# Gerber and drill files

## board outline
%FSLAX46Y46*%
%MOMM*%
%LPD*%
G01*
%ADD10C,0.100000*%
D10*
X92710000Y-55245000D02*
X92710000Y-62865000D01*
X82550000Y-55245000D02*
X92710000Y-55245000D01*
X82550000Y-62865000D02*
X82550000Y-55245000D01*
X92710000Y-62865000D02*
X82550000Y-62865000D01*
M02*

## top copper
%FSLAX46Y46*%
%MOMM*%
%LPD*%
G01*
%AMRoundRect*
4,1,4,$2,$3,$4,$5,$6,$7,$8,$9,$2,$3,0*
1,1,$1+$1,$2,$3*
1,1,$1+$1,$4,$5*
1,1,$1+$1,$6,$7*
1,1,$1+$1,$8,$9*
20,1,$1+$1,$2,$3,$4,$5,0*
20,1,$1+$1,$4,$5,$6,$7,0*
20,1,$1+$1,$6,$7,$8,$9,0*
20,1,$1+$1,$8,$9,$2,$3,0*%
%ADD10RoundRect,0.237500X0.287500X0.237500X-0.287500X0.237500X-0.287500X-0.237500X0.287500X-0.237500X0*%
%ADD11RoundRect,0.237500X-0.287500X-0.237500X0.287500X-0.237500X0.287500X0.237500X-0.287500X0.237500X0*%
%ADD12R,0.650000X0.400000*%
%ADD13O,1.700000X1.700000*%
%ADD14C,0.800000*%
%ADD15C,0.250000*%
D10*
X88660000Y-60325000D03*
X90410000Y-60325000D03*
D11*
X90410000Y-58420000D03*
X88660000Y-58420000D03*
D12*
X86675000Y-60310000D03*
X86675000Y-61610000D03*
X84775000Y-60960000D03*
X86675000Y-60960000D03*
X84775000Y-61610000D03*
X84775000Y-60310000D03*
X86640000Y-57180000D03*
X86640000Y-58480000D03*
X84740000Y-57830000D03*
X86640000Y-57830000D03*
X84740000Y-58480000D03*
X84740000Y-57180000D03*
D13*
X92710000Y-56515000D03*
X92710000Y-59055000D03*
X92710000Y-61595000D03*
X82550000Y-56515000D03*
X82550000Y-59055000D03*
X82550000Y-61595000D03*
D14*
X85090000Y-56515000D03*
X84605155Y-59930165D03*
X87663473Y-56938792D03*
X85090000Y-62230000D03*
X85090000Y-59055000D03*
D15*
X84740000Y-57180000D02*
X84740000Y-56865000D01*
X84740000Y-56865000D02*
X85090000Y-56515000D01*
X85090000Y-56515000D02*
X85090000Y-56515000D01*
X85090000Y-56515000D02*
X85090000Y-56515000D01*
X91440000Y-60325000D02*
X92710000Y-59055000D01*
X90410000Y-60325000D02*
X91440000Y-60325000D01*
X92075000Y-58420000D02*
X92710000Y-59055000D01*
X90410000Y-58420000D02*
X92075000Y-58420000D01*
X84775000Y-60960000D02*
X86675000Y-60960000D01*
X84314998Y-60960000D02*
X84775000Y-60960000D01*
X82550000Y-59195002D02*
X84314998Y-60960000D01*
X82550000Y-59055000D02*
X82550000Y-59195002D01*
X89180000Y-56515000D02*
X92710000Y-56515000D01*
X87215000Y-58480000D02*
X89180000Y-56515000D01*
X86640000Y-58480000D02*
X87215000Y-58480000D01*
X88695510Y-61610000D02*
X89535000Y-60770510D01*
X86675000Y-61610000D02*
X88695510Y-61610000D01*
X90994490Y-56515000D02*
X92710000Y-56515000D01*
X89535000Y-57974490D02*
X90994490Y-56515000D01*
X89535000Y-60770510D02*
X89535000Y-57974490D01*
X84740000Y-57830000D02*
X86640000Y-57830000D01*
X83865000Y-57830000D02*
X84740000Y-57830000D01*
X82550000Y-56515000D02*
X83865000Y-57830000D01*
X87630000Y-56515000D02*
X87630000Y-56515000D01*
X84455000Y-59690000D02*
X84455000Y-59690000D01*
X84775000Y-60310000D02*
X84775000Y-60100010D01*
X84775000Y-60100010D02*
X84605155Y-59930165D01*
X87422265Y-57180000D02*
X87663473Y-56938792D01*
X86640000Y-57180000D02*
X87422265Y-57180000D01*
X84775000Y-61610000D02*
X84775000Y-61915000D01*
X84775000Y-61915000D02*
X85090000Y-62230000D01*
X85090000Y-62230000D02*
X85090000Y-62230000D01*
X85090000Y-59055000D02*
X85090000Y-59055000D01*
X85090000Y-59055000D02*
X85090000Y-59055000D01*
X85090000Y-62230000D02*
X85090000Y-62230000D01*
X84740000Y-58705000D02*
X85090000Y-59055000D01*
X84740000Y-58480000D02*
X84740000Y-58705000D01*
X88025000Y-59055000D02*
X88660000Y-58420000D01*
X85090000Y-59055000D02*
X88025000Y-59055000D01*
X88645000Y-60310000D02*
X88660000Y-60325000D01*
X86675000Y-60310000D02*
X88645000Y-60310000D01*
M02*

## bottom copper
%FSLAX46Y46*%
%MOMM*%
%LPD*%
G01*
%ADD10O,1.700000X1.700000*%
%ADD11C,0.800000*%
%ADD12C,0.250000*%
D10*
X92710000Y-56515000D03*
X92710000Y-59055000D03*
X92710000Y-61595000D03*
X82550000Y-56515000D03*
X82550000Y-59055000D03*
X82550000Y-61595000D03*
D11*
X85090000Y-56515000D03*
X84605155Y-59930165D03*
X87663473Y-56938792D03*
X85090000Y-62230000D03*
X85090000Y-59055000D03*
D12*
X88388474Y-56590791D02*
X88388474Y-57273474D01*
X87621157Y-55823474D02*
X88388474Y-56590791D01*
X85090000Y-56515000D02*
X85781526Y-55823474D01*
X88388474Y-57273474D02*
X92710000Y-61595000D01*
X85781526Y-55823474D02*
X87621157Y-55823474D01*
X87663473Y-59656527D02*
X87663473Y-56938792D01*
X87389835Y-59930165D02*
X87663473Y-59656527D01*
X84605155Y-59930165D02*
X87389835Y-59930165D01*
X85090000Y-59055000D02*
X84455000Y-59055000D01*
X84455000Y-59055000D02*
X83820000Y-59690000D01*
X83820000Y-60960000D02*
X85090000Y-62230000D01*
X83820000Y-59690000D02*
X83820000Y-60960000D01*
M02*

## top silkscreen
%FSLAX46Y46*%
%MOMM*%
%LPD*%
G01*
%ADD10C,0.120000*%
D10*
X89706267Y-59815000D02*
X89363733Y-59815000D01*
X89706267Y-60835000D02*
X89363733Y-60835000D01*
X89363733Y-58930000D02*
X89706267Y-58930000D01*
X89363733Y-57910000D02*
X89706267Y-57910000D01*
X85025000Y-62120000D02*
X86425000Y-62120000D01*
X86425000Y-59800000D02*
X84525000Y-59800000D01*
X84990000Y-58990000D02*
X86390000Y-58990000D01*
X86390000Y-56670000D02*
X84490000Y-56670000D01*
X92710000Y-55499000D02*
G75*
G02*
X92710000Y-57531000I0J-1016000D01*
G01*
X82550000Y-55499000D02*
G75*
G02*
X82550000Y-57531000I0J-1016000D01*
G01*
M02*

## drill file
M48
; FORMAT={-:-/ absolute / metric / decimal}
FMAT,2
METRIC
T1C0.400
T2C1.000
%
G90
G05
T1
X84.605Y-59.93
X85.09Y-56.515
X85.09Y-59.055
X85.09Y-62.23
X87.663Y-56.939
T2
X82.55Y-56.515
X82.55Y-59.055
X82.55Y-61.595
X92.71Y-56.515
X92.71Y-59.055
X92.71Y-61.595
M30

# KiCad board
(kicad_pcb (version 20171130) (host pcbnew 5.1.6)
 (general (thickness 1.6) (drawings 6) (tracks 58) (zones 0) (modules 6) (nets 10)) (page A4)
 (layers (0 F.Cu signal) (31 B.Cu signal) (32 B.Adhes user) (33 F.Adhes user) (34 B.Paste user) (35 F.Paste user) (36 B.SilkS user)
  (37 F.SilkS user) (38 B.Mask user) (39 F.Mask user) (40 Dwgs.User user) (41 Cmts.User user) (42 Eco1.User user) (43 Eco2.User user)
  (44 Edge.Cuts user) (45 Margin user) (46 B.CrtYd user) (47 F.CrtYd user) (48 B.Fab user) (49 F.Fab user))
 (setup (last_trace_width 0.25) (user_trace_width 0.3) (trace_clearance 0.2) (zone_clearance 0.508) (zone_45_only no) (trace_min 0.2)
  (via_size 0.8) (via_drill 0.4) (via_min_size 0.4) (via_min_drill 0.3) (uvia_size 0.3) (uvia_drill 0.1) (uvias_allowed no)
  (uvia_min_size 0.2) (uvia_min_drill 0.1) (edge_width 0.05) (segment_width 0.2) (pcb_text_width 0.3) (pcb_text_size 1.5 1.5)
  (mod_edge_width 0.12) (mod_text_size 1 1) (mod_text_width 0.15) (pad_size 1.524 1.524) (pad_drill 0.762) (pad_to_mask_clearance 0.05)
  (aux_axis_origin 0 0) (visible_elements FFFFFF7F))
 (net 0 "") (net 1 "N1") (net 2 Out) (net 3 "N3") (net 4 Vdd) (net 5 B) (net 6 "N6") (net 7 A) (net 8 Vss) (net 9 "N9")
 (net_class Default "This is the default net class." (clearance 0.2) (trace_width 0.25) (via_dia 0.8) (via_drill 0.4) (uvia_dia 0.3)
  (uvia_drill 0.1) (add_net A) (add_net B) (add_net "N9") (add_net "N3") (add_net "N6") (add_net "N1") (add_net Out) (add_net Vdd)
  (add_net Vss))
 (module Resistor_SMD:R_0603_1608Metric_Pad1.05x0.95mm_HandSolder (layer F.Cu) (at 89.535 60.325 180)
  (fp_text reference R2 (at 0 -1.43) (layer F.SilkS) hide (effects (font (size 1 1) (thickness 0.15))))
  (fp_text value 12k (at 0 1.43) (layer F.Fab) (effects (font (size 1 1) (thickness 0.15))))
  (fp_line (start -0.171267 0.51) (end 0.171267 0.51) (layer F.SilkS) (width 0.12))
  (fp_line (start -0.171267 -0.51) (end 0.171267 -0.51) (layer F.SilkS) (width 0.12))
  (pad 2 smd roundrect (at 0.875 0 180) (size 1.05 0.95) (layers F.Cu F.Paste F.Mask) (roundrect_rratio 0.25) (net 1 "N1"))
  (pad 1 smd roundrect (at -0.875 0 180) (size 1.05 0.95) (layers F.Cu F.Paste F.Mask) (roundrect_rratio 0.25) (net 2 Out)))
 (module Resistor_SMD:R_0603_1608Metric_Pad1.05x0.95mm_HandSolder (layer F.Cu) (at 89.535 58.42)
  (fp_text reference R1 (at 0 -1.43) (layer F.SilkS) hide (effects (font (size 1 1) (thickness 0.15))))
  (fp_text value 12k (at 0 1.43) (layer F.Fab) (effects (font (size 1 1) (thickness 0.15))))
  (fp_line (start -0.171267 0.51) (end 0.171267 0.51) (layer F.SilkS) (width 0.12))
  (fp_line (start -0.171267 -0.51) (end 0.171267 -0.51) (layer F.SilkS) (width 0.12))
  (pad 2 smd roundrect (at 0.875 0) (size 1.05 0.95) (layers F.Cu F.Paste F.Mask) (roundrect_rratio 0.25) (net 2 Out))
  (pad 1 smd roundrect (at -0.875 0) (size 1.05 0.95) (layers F.Cu F.Paste F.Mask) (roundrect_rratio 0.25) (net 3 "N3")))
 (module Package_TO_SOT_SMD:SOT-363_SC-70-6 (layer F.Cu) (at 85.725 60.96)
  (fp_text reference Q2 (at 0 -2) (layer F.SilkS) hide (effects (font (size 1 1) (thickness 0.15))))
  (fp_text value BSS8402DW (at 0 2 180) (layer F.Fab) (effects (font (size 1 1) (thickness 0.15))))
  (fp_line (start -0.7 1.16) (end 0.7 1.16) (layer F.SilkS) (width 0.12))
  (fp_line (start 0.7 -1.16) (end -1.2 -1.16) (layer F.SilkS) (width 0.12))
  (pad 6 smd rect (at 0.95 -0.65) (size 0.65 0.4) (layers F.Cu F.Paste F.Mask) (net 1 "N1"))
  (pad 4 smd rect (at 0.95 0.65) (size 0.65 0.4) (layers F.Cu F.Paste F.Mask) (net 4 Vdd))
  (pad 2 smd rect (at -0.95 0) (size 0.65 0.4) (layers F.Cu F.Paste F.Mask) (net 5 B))
  (pad 5 smd rect (at 0.95 0) (size 0.65 0.4) (layers F.Cu F.Paste F.Mask) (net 5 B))
  (pad 3 smd rect (at -0.95 0.65) (size 0.65 0.4) (layers F.Cu F.Paste F.Mask) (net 3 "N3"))
  (pad 1 smd rect (at -0.95 -0.65) (size 0.65 0.4) (layers F.Cu F.Paste F.Mask) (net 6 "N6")))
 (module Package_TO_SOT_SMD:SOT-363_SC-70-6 (layer F.Cu) (at 85.69 57.83)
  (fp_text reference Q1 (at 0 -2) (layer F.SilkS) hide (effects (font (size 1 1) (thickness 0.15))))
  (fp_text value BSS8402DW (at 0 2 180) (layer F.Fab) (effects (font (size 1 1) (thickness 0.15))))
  (fp_line (start -0.7 1.16) (end 0.7 1.16) (layer F.SilkS) (width 0.12))
  (fp_line (start 0.7 -1.16) (end -1.2 -1.16) (layer F.SilkS) (width 0.12))
  (pad 6 smd rect (at 0.95 -0.65) (size 0.65 0.4) (layers F.Cu F.Paste F.Mask) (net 6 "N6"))
  (pad 4 smd rect (at 0.95 0.65) (size 0.65 0.4) (layers F.Cu F.Paste F.Mask) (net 4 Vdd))
  (pad 2 smd rect (at -0.95 0) (size 0.65 0.4) (layers F.Cu F.Paste F.Mask) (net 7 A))
  (pad 5 smd rect (at 0.95 0) (size 0.65 0.4) (layers F.Cu F.Paste F.Mask) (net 7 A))
  (pad 3 smd rect (at -0.95 0.65) (size 0.65 0.4) (layers F.Cu F.Paste F.Mask) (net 3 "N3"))
  (pad 1 smd rect (at -0.95 -0.65) (size 0.65 0.4) (layers F.Cu F.Paste F.Mask) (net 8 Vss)))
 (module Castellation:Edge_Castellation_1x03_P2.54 (layer F.Cu) (at 92.71 56.515)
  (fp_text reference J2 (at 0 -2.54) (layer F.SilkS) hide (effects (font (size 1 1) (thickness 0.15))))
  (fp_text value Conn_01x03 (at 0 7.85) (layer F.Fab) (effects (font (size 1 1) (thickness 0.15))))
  (fp_arc (start 0 0) (end 0 1.016) (angle -180) (layer F.SilkS) (width 0.12))
  (pad 1 thru_hole oval (at 0 0) (size 1.7 1.7) (drill 1) (layers *.Cu *.Mask) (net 4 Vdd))
  (pad 2 thru_hole oval (at 0 2.54) (size 1.7 1.7) (drill 1) (layers *.Cu *.Mask) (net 2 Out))
  (pad 3 thru_hole oval (at 0 5.08) (size 1.7 1.7) (drill 1) (layers *.Cu *.Mask) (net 8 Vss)))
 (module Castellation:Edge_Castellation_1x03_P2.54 (layer F.Cu) (at 82.55 56.515)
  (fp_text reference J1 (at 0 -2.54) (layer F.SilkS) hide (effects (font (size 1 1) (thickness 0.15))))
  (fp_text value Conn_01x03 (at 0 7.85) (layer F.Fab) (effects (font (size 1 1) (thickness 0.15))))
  (fp_arc (start 0 0) (end 0 1.016) (angle -180) (layer F.SilkS) (width 0.12))
  (pad 1 thru_hole oval (at 0 0) (size 1.7 1.7) (drill 1) (layers *.Cu *.Mask) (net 7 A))
  (pad 2 thru_hole oval (at 0 2.54) (size 1.7 1.7) (drill 1) (layers *.Cu *.Mask) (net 5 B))
  (pad 3 thru_hole oval (at 0 5.08) (size 1.7 1.7) (drill 1) (layers *.Cu *.Mask) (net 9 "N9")))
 (gr_line (start 92.71 55.245) (end 92.71 62.865) (layer Edge.Cuts) (width 0.1))
 (gr_line (start 82.55 55.245) (end 92.71 55.245) (layer Edge.Cuts) (width 0.1))
 (gr_line (start 82.55 62.865) (end 82.55 55.245) (layer Edge.Cuts) (width 0.1))
 (gr_line (start 92.71 62.865) (end 82.55 62.865) (layer Edge.Cuts) (width 0.1))
 (segment (start 84.74 57.18) (end 84.74 56.865) (width 0.25) (layer F.Cu) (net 8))
 (segment (start 84.74 56.865) (end 85.09 56.515) (width 0.25) (layer F.Cu) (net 8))
 (segment (start 85.09 56.515) (end 85.09 56.515) (width 0.25) (layer F.Cu) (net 8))
 (segment (start 85.09 56.515) (end 85.09 56.515) (width 0.25) (layer F.Cu) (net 8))
 (via (at 85.09 56.515) (size 0.8) (drill 0.4) (layers F.Cu B.Cu) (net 8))
 (segment (start 88.388474 56.590791) (end 88.388474 57.273474) (width 0.25) (layer B.Cu) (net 8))
 (segment (start 87.621157 55.823474) (end 88.388474 56.590791) (width 0.25) (layer B.Cu) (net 8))
 (segment (start 85.09 56.515) (end 85.781526 55.823474) (width 0.25) (layer B.Cu) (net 8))
 (segment (start 88.388474 57.273474) (end 92.71 61.595) (width 0.25) (layer B.Cu) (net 8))
 (segment (start 85.781526 55.823474) (end 87.621157 55.823474) (width 0.25) (layer B.Cu) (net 8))
 (segment (start 91.44 60.325) (end 92.71 59.055) (width 0.25) (layer F.Cu) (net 2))
 (segment (start 90.41 60.325) (end 91.44 60.325) (width 0.25) (layer F.Cu) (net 2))
 (segment (start 92.075 58.42) (end 92.71 59.055) (width 0.25) (layer F.Cu) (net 2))
 (segment (start 90.41 58.42) (end 92.075 58.42) (width 0.25) (layer F.Cu) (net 2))
 (segment (start 84.775 60.96) (end 86.675 60.96) (width 0.25) (layer F.Cu) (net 5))
 (segment (start 84.314998 60.96) (end 84.775 60.96) (width 0.25) (layer F.Cu) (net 5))
 (segment (start 82.55 59.195002) (end 84.314998 60.96) (width 0.25) (layer F.Cu) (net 5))
 (segment (start 82.55 59.055) (end 82.55 59.195002) (width 0.25) (layer F.Cu) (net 5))
 (segment (start 89.18 56.515) (end 92.71 56.515) (width 0.25) (layer F.Cu) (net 4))
 (segment (start 87.215 58.48) (end 89.18 56.515) (width 0.25) (layer F.Cu) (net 4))
 (segment (start 86.64 58.48) (end 87.215 58.48) (width 0.25) (layer F.Cu) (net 4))
 (segment (start 88.69551 61.61) (end 89.535 60.77051) (width 0.25) (layer F.Cu) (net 4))
 (segment (start 86.675 61.61) (end 88.69551 61.61) (width 0.25) (layer F.Cu) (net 4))
 (segment (start 90.99449 56.515) (end 92.71 56.515) (width 0.25) (layer F.Cu) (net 4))
 (segment (start 89.535 57.97449) (end 90.99449 56.515) (width 0.25) (layer F.Cu) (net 4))
 (segment (start 89.535 60.77051) (end 89.535 57.97449) (width 0.25) (layer F.Cu) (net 4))
 (segment (start 84.74 57.83) (end 86.64 57.83) (width 0.25) (layer F.Cu) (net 7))
 (segment (start 83.865 57.83) (end 84.74 57.83) (width 0.25) (layer F.Cu) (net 7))
 (segment (start 82.55 56.515) (end 83.865 57.83) (width 0.25) (layer F.Cu) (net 7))
 (segment (start 87.63 56.515) (end 87.63 56.515) (width 0.25) (layer F.Cu) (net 6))
 (segment (start 84.455 59.69) (end 84.455 59.69) (width 0.25) (layer F.Cu) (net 6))
 (segment (start 84.775 60.31) (end 84.775 60.10001) (width 0.25) (layer F.Cu) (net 6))
 (segment (start 84.775 60.10001) (end 84.605155 59.930165) (width 0.25) (layer F.Cu) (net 6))
 (via (at 84.605155 59.930165) (size 0.8) (drill 0.4) (layers F.Cu B.Cu) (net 6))
 (segment (start 87.663473 59.656527) (end 87.663473 56.938792) (width 0.25) (layer B.Cu) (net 6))
 (segment (start 87.422265 57.18) (end 87.663473 56.938792) (width 0.25) (layer F.Cu) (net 6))
 (via (at 87.663473 56.938792) (size 0.8) (drill 0.4) (layers F.Cu B.Cu) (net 6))
 (segment (start 86.64 57.18) (end 87.422265 57.18) (width 0.25) (layer F.Cu) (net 6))
 (segment (start 87.389835 59.930165) (end 87.663473 59.656527) (width 0.25) (layer B.Cu) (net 6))
 (segment (start 84.605155 59.930165) (end 87.389835 59.930165) (width 0.25) (layer B.Cu) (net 6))
 (segment (start 84.775 61.61) (end 84.775 61.915) (width 0.25) (layer F.Cu) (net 3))
 (segment (start 84.775 61.915) (end 85.09 62.23) (width 0.25) (layer F.Cu) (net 3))
 (segment (start 85.09 62.23) (end 85.09 62.23) (width 0.25) (layer F.Cu) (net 3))
 (segment (start 85.09 59.055) (end 85.09 59.055) (width 0.25) (layer F.Cu) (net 3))
 (segment (start 85.09 59.055) (end 85.09 59.055) (width 0.25) (layer F.Cu) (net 3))
 (segment (start 85.09 62.23) (end 85.09 62.23) (width 0.25) (layer F.Cu) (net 3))
 (via (at 85.09 62.23) (size 0.8) (drill 0.4) (layers F.Cu B.Cu) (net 3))
 (segment (start 84.74 58.705) (end 85.09 59.055) (width 0.25) (layer F.Cu) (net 3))
 (segment (start 84.74 58.48) (end 84.74 58.705) (width 0.25) (layer F.Cu) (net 3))
 (segment (start 88.025 59.055) (end 88.66 58.42) (width 0.25) (layer F.Cu) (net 3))
 (via (at 85.09 59.055) (size 0.8) (drill 0.4) (layers F.Cu B.Cu) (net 3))
 (segment (start 85.09 59.055) (end 88.025 59.055) (width 0.25) (layer F.Cu) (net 3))
 (segment (start 85.09 59.055) (end 84.455 59.055) (width 0.25) (layer B.Cu) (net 3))
 (segment (start 84.455 59.055) (end 83.82 59.69) (width 0.25) (layer B.Cu) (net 3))
 (segment (start 83.82 60.96) (end 85.09 62.23) (width 0.25) (layer B.Cu) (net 3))
 (segment (start 83.82 59.69) (end 83.82 60.96) (width 0.25) (layer B.Cu) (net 3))
 (segment (start 88.645 60.31) (end 88.66 60.325) (width 0.25) (layer F.Cu) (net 1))
 (segment (start 86.675 60.31) (end 88.645 60.31) (width 0.25) (layer F.Cu) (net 1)))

